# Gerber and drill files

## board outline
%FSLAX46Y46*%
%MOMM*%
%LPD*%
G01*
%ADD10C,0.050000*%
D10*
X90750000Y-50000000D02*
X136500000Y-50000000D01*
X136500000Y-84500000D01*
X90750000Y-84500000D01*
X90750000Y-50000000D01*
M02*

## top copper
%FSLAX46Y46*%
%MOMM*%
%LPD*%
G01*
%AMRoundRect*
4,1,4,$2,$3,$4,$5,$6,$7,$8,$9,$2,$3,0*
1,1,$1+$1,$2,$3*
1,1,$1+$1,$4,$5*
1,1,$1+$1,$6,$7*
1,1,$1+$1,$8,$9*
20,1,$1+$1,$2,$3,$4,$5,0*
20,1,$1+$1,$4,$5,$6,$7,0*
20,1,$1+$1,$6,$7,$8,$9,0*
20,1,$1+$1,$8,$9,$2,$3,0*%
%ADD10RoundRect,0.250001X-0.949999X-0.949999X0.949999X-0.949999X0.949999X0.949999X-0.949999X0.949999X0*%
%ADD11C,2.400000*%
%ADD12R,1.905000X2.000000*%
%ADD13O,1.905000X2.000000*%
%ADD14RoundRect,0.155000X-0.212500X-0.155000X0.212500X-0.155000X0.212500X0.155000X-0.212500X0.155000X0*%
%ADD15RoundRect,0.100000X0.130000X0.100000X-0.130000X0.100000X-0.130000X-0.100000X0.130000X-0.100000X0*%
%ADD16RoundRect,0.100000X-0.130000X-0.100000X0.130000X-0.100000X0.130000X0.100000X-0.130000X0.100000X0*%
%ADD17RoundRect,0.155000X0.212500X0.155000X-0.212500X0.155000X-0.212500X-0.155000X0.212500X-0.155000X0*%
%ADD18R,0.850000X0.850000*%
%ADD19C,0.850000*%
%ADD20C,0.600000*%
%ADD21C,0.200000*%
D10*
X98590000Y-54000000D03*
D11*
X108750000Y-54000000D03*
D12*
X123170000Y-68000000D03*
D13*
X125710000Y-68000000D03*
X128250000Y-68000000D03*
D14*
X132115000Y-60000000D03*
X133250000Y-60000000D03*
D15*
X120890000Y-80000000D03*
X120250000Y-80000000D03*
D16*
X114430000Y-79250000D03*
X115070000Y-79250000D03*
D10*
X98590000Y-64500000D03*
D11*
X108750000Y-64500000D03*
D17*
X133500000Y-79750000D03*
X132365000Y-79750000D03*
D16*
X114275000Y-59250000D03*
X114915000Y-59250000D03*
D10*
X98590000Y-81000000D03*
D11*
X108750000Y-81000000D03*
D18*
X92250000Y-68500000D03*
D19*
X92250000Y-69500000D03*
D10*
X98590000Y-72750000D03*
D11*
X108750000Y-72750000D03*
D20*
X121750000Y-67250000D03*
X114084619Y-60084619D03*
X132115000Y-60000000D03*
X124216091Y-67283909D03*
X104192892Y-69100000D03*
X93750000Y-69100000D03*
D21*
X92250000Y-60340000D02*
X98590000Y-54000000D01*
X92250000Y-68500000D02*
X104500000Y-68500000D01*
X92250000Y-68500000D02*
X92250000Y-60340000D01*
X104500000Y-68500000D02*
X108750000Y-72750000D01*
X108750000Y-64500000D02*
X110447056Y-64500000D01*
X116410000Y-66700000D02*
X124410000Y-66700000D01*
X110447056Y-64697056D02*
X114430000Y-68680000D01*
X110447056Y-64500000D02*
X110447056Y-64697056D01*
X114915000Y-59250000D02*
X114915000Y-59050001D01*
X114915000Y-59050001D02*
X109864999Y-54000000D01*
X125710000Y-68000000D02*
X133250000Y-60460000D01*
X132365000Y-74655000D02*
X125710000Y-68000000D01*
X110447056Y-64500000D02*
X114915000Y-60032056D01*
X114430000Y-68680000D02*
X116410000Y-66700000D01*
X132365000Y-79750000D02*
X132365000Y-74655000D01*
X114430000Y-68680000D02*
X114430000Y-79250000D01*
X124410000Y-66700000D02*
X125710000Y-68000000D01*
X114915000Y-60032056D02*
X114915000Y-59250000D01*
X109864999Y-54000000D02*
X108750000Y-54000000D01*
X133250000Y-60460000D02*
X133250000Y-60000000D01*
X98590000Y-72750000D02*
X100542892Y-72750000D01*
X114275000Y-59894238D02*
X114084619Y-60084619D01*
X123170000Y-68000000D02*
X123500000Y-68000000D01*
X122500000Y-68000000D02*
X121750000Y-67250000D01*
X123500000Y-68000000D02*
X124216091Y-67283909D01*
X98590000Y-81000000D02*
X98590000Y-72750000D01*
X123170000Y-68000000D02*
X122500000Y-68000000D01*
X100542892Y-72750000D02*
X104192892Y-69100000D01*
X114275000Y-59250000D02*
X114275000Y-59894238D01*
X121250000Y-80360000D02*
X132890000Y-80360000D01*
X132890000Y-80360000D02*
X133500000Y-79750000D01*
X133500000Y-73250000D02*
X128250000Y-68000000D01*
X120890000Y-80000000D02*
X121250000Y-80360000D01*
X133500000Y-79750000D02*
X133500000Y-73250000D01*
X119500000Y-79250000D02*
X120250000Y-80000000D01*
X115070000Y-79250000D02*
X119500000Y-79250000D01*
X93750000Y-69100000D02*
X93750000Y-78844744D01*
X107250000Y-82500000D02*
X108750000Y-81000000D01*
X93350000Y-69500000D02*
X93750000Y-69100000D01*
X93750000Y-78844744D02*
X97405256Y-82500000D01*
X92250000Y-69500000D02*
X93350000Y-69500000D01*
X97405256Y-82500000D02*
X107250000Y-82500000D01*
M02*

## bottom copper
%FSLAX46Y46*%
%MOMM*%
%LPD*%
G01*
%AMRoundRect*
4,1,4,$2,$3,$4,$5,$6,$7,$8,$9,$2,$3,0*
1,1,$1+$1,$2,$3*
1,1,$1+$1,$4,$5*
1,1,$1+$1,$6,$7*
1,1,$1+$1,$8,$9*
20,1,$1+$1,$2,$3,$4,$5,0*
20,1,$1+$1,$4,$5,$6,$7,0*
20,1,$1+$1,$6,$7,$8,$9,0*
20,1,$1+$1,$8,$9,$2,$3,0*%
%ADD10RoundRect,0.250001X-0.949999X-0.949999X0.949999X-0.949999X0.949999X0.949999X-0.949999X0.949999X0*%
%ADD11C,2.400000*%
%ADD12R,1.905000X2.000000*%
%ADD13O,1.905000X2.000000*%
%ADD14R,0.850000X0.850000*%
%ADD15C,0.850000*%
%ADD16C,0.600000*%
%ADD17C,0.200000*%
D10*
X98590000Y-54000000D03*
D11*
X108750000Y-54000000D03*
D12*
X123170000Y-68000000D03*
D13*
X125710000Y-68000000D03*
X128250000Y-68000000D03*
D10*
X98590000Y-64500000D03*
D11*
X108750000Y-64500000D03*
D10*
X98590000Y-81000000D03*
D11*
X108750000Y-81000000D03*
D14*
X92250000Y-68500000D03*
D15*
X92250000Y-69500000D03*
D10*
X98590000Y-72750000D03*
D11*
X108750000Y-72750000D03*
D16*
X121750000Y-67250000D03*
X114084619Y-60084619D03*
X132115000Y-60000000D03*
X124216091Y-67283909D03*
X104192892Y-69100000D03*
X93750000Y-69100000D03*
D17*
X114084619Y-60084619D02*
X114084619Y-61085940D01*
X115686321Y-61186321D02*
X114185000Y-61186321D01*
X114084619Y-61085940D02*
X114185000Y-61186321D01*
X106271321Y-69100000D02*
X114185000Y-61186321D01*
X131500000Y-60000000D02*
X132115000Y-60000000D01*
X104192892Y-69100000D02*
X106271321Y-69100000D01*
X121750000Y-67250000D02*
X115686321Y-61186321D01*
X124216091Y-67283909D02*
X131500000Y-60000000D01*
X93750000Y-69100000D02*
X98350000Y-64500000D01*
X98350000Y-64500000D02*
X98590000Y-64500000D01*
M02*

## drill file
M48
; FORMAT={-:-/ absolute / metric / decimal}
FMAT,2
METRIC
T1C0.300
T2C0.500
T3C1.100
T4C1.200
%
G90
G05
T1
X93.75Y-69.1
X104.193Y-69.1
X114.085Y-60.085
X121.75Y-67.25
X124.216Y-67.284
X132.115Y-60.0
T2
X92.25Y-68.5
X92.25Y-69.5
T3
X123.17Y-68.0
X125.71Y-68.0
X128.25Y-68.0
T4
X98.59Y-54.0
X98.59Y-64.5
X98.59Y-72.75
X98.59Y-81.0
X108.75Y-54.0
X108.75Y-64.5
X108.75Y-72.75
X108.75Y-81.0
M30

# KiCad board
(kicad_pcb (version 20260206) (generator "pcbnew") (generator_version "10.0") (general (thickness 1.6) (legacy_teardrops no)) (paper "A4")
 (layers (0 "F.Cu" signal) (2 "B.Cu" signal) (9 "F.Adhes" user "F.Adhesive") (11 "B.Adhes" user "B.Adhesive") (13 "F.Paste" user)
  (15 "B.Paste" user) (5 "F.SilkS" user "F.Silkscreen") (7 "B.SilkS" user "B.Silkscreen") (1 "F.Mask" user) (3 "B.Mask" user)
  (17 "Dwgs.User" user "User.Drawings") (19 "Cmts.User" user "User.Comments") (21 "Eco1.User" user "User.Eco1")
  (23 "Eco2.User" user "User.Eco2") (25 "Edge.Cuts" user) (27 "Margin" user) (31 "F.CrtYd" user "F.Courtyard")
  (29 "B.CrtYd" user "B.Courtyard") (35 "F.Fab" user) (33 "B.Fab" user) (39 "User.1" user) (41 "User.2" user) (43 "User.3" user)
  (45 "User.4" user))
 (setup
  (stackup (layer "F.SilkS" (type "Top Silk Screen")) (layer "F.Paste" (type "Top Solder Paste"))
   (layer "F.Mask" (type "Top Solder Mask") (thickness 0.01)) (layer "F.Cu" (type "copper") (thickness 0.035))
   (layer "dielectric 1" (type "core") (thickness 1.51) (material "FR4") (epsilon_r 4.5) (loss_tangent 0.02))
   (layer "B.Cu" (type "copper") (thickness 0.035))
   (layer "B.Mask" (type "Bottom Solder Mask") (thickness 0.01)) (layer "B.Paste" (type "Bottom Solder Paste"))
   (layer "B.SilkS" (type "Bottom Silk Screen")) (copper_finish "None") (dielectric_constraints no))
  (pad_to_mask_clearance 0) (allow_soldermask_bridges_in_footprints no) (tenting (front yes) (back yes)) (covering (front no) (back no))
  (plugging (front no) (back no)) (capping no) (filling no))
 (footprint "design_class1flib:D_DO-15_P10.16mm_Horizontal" (layer "F.Cu") (at 98.59 54)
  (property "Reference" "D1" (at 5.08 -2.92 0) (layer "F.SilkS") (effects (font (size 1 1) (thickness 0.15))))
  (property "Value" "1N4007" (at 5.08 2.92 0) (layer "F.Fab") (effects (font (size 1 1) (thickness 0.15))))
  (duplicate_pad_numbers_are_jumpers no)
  (pad "1" thru_hole roundrect (at 0 0) (size 2.4 2.4) (drill 1.2) (layers "*.Cu" "*.Mask") (remove_unused_layers no)
   (roundrect_rratio 0.104167) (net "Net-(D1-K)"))
  (pad "2" thru_hole circle (at 10.16 0) (size 2.4 2.4) (drill 1.2) (layers "*.Cu" "*.Mask") (remove_unused_layers no) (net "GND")))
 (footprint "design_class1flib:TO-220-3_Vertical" (layer "F.Cu") (at 123.17 68)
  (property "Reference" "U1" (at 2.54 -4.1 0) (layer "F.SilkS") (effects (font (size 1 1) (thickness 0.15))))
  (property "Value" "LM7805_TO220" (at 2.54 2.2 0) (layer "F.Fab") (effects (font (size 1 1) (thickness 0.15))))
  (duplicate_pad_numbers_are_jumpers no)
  (pad "1" thru_hole rect (at 0 0) (size 1.905 2) (drill 1.1) (layers "*.Cu" "*.Mask") (remove_unused_layers no) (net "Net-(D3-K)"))
  (pad "2" thru_hole oval (at 2.54 0) (size 1.905 2) (drill 1.1) (layers "*.Cu" "*.Mask") (remove_unused_layers no) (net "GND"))
  (pad "3" thru_hole oval (at 5.08 0) (size 1.905 2) (drill 1.1) (layers "*.Cu" "*.Mask") (remove_unused_layers no) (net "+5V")))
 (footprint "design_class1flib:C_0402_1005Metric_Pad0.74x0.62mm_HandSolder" (layer "F.Cu") (at 132.6825 60)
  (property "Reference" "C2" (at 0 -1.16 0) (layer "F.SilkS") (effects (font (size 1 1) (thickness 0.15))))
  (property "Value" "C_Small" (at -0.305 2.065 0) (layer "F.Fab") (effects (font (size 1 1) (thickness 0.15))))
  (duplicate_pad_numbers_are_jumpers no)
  (pad "1" smd roundrect (at -0.5675 0) (size 0.735 0.62) (layers "F.Cu" "F.Mask" "F.Paste") (roundrect_rratio 0.25) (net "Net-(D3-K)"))
  (pad "2" smd roundrect (at 0.5675 0) (size 0.735 0.62) (layers "F.Cu" "F.Mask" "F.Paste") (roundrect_rratio 0.25) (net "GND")))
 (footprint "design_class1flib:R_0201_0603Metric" (layer "F.Cu") (at 120.57 80 180)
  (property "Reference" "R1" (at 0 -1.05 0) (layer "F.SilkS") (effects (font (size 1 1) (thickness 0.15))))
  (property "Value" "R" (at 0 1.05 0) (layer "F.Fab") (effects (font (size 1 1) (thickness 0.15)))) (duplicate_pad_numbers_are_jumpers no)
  (pad "" smd roundrect (at -0.345 0 180) (size 0.318 0.36) (layers "F.Paste") (roundrect_rratio 0.25))
  (pad "" smd roundrect (at 0.345 0 180) (size 0.318 0.36) (layers "F.Paste") (roundrect_rratio 0.25))
  (pad "1" smd roundrect (at -0.32 0 180) (size 0.46 0.4) (layers "F.Cu" "F.Mask") (roundrect_rratio 0.25) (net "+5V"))
  (pad "2" smd roundrect (at 0.32 0 180) (size 0.46 0.4) (layers "F.Cu" "F.Mask") (roundrect_rratio 0.25) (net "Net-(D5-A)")))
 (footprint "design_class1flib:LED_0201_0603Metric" (layer "F.Cu") (at 114.75 79.25)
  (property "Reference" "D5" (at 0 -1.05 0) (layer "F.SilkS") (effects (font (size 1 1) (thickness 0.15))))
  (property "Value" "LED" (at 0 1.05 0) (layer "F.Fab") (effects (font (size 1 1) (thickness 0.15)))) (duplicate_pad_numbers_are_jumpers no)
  (pad "" smd roundrect (at -0.345 0) (size 0.318 0.36) (layers "F.Paste") (roundrect_rratio 0.25))
  (pad "" smd roundrect (at 0.345 0) (size 0.318 0.36) (layers "F.Paste") (roundrect_rratio 0.25))
  (pad "1" smd roundrect (at -0.32 0) (size 0.46 0.4) (layers "F.Cu" "F.Mask") (roundrect_rratio 0.25) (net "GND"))
  (pad "2" smd roundrect (at 0.32 0) (size 0.46 0.4) (layers "F.Cu" "F.Mask") (roundrect_rratio 0.25) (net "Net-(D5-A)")))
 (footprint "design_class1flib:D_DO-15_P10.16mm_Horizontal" (layer "F.Cu") (at 98.59 64.5)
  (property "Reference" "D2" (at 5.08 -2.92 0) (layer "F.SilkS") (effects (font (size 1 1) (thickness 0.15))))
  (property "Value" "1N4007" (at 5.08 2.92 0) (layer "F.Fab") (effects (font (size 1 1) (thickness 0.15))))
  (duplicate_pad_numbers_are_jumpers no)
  (pad "1" thru_hole roundrect (at 0 0) (size 2.4 2.4) (drill 1.2) (layers "*.Cu" "*.Mask") (remove_unused_layers no)
   (roundrect_rratio 0.104167) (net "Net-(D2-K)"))
  (pad "2" thru_hole circle (at 10.16 0) (size 2.4 2.4) (drill 1.2) (layers "*.Cu" "*.Mask") (remove_unused_layers no) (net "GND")))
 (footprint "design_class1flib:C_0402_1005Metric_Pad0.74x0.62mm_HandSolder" (layer "F.Cu") (at 132.9325 79.75 180)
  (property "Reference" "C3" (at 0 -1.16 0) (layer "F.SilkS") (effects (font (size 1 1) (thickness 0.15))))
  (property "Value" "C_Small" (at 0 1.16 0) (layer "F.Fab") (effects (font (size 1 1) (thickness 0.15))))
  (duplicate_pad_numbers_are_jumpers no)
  (pad "1" smd roundrect (at -0.5675 0 180) (size 0.735 0.62) (layers "F.Cu" "F.Mask" "F.Paste") (roundrect_rratio 0.25) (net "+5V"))
  (pad "2" smd roundrect (at 0.5675 0 180) (size 0.735 0.62) (layers "F.Cu" "F.Mask" "F.Paste") (roundrect_rratio 0.25) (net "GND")))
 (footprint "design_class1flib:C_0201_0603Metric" (layer "F.Cu") (at 114.595 59.25)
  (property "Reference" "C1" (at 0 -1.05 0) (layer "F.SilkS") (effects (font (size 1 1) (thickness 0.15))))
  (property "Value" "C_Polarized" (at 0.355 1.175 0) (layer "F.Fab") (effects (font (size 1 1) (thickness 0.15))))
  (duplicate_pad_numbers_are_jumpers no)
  (pad "" smd roundrect (at -0.345 0) (size 0.318 0.36) (layers "F.Paste") (roundrect_rratio 0.25))
  (pad "" smd roundrect (at 0.345 0) (size 0.318 0.36) (layers "F.Paste") (roundrect_rratio 0.25))
  (pad "1" smd roundrect (at -0.32 0) (size 0.46 0.4) (layers "F.Cu" "F.Mask") (roundrect_rratio 0.25) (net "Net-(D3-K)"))
  (pad "2" smd roundrect (at 0.32 0) (size 0.46 0.4) (layers "F.Cu" "F.Mask") (roundrect_rratio 0.25) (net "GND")))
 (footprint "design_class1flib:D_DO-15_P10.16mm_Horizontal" (layer "F.Cu") (at 98.59 81)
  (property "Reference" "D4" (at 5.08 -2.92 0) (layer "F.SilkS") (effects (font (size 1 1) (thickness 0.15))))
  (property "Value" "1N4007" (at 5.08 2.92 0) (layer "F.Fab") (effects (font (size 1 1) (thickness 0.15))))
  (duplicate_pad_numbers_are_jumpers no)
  (pad "1" thru_hole roundrect (at 0 0) (size 2.4 2.4) (drill 1.2) (layers "*.Cu" "*.Mask") (remove_unused_layers no)
   (roundrect_rratio 0.104167) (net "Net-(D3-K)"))
  (pad "2" thru_hole circle (at 10.16 0) (size 2.4 2.4) (drill 1.2) (layers "*.Cu" "*.Mask") (remove_unused_layers no) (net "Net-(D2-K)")))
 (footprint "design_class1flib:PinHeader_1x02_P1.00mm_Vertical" (layer "F.Cu") (at 92.25 68.5)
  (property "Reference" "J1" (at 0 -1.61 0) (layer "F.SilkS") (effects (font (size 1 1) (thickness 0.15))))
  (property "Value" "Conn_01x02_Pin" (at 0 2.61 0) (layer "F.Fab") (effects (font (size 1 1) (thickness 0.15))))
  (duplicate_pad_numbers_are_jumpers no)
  (pad "1" thru_hole rect (at 0 0) (size 0.85 0.85) (drill 0.5) (layers "*.Cu" "*.Mask") (remove_unused_layers no) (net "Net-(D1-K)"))
  (pad "2" thru_hole circle (at 0 1) (size 0.85 0.85) (drill 0.5) (layers "*.Cu" "*.Mask") (remove_unused_layers no) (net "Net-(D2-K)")))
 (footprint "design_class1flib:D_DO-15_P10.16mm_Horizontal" (layer "F.Cu") (at 98.59 72.75)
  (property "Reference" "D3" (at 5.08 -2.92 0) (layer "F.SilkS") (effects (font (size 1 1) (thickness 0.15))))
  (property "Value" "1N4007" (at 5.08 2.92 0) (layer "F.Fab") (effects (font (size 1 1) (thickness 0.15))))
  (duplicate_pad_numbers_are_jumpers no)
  (pad "1" thru_hole roundrect (at 0 0) (size 2.4 2.4) (drill 1.2) (layers "*.Cu" "*.Mask") (remove_unused_layers no)
   (roundrect_rratio 0.104167) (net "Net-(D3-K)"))
  (pad "2" thru_hole circle (at 10.16 0) (size 2.4 2.4) (drill 1.2) (layers "*.Cu" "*.Mask") (remove_unused_layers no) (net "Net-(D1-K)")))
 (gr_rect (start 90.75 50) (end 136.5 84.5) (stroke (width 0.05) (type default)) (fill no) (layer "Edge.Cuts"))
 (segment (start 92.25 60.34) (end 98.59 54) (width 0.2) (layer "F.Cu") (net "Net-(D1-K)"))
 (segment (start 92.25 68.5) (end 104.5 68.5) (width 0.2) (layer "F.Cu") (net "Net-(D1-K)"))
 (segment (start 92.25 68.5) (end 92.25 60.34) (width 0.2) (layer "F.Cu") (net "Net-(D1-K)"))
 (segment (start 104.5 68.5) (end 108.75 72.75) (width 0.2) (layer "F.Cu") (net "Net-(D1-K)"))
 (segment (start 108.75 64.5) (end 110.447056 64.5) (width 0.2) (layer "F.Cu") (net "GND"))
 (segment (start 116.41 66.7) (end 124.41 66.7) (width 0.2) (layer "F.Cu") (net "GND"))
 (segment (start 110.447056 64.697056) (end 114.43 68.68) (width 0.2) (layer "F.Cu") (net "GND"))
 (segment (start 110.447056 64.5) (end 110.447056 64.697056) (width 0.2) (layer "F.Cu") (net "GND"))
 (segment (start 114.915 59.25) (end 114.915 59.050001) (width 0.2) (layer "F.Cu") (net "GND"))
 (segment (start 114.915 59.050001) (end 109.864999 54) (width 0.2) (layer "F.Cu") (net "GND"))
 (segment (start 125.71 68) (end 133.25 60.46) (width 0.2) (layer "F.Cu") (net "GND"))
 (segment (start 132.365 74.655) (end 125.71 68) (width 0.2) (layer "F.Cu") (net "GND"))
 (segment (start 110.447056 64.5) (end 114.915 60.032056) (width 0.2) (layer "F.Cu") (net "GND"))
 (segment (start 114.43 68.68) (end 116.41 66.7) (width 0.2) (layer "F.Cu") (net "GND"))
 (segment (start 132.365 79.75) (end 132.365 74.655) (width 0.2) (layer "F.Cu") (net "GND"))
 (segment (start 114.43 68.68) (end 114.43 79.25) (width 0.2) (layer "F.Cu") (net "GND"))
 (segment (start 124.41 66.7) (end 125.71 68) (width 0.2) (layer "F.Cu") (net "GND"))
 (segment (start 114.915 60.032056) (end 114.915 59.25) (width 0.2) (layer "F.Cu") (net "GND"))
 (segment (start 109.864999 54) (end 108.75 54) (width 0.2) (layer "F.Cu") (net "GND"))
 (segment (start 133.25 60.46) (end 133.25 60) (width 0.2) (layer "F.Cu") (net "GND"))
 (segment (start 98.59 72.75) (end 100.542892 72.75) (width 0.2) (layer "F.Cu") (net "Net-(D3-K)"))
 (segment (start 114.275 59.894238) (end 114.084619 60.084619) (width 0.2) (layer "F.Cu") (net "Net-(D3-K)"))
 (segment (start 123.17 68) (end 123.5 68) (width 0.2) (layer "F.Cu") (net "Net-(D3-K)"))
 (segment (start 122.5 68) (end 121.75 67.25) (width 0.2) (layer "F.Cu") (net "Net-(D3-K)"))
 (segment (start 123.5 68) (end 124.216091 67.283909) (width 0.2) (layer "F.Cu") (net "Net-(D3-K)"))
 (segment (start 98.59 81) (end 98.59 72.75) (width 0.2) (layer "F.Cu") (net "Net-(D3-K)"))
 (segment (start 123.17 68) (end 122.5 68) (width 0.2) (layer "F.Cu") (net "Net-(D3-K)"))
 (segment (start 100.542892 72.75) (end 104.192892 69.1) (width 0.2) (layer "F.Cu") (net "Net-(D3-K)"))
 (segment (start 114.275 59.25) (end 114.275 59.894238) (width 0.2) (layer "F.Cu") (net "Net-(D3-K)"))
 (via (at 121.75 67.25) (size 0.6) (drill 0.3) (layers "F.Cu" "B.Cu") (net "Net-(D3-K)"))
 (via (at 114.084619 60.084619) (size 0.6) (drill 0.3) (layers "F.Cu" "B.Cu") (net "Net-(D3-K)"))
 (via (at 132.115 60) (size 0.6) (drill 0.3) (layers "F.Cu" "B.Cu") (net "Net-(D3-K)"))
 (via (at 124.216091 67.283909) (size 0.6) (drill 0.3) (layers "F.Cu" "B.Cu") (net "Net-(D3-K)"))
 (via (at 104.192892 69.1) (size 0.6) (drill 0.3) (layers "F.Cu" "B.Cu") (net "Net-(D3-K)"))
 (segment (start 114.084619 60.084619) (end 114.084619 61.08594) (width 0.2) (layer "B.Cu") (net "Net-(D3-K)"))
 (segment (start 115.686321 61.186321) (end 114.185 61.186321) (width 0.2) (layer "B.Cu") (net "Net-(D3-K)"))
 (segment (start 114.084619 61.08594) (end 114.185 61.186321) (width 0.2) (layer "B.Cu") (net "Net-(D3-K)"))
 (segment (start 106.271321 69.1) (end 114.185 61.186321) (width 0.2) (layer "B.Cu") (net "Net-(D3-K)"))
 (segment (start 131.5 60) (end 132.115 60) (width 0.2) (layer "B.Cu") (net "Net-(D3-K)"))
 (segment (start 104.192892 69.1) (end 106.271321 69.1) (width 0.2) (layer "B.Cu") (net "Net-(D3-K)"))
 (segment (start 121.75 67.25) (end 115.686321 61.186321) (width 0.2) (layer "B.Cu") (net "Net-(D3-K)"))
 (segment (start 124.216091 67.283909) (end 131.5 60) (width 0.2) (layer "B.Cu") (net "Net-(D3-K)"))
 (segment (start 121.25 80.36) (end 132.89 80.36) (width 0.2) (layer "F.Cu") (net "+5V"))
 (segment (start 132.89 80.36) (end 133.5 79.75) (width 0.2) (layer "F.Cu") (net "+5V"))
 (segment (start 133.5 73.25) (end 128.25 68) (width 0.2) (layer "F.Cu") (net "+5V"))
 (segment (start 120.89 80) (end 121.25 80.36) (width 0.2) (layer "F.Cu") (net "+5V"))
 (segment (start 133.5 79.75) (end 133.5 73.25) (width 0.2) (layer "F.Cu") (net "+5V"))
 (segment (start 119.5 79.25) (end 120.25 80) (width 0.2) (layer "F.Cu") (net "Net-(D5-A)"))
 (segment (start 115.07 79.25) (end 119.5 79.25) (width 0.2) (layer "F.Cu") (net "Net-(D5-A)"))
 (segment (start 93.75 69.1) (end 93.75 78.844744) (width 0.2) (layer "F.Cu") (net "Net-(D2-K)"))
 (segment (start 107.25 82.5) (end 108.75 81) (width 0.2) (layer "F.Cu") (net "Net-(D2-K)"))
 (segment (start 93.35 69.5) (end 93.75 69.1) (width 0.2) (layer "F.Cu") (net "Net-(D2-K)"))
 (segment (start 93.75 78.844744) (end 97.405256 82.5) (width 0.2) (layer "F.Cu") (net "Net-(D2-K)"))
 (segment (start 92.25 69.5) (end 93.35 69.5) (width 0.2) (layer "F.Cu") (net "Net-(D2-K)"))
 (segment (start 97.405256 82.5) (end 107.25 82.5) (width 0.2) (layer "F.Cu") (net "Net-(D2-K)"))
 (via (at 93.75 69.1) (size 0.6) (drill 0.3) (layers "F.Cu" "B.Cu") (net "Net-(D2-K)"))
 (segment (start 93.75 69.1) (end 98.35 64.5) (width 0.2) (layer "B.Cu") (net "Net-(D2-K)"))
 (segment (start 98.35 64.5) (end 98.59 64.5) (width 0.2) (layer "B.Cu") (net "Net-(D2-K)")))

